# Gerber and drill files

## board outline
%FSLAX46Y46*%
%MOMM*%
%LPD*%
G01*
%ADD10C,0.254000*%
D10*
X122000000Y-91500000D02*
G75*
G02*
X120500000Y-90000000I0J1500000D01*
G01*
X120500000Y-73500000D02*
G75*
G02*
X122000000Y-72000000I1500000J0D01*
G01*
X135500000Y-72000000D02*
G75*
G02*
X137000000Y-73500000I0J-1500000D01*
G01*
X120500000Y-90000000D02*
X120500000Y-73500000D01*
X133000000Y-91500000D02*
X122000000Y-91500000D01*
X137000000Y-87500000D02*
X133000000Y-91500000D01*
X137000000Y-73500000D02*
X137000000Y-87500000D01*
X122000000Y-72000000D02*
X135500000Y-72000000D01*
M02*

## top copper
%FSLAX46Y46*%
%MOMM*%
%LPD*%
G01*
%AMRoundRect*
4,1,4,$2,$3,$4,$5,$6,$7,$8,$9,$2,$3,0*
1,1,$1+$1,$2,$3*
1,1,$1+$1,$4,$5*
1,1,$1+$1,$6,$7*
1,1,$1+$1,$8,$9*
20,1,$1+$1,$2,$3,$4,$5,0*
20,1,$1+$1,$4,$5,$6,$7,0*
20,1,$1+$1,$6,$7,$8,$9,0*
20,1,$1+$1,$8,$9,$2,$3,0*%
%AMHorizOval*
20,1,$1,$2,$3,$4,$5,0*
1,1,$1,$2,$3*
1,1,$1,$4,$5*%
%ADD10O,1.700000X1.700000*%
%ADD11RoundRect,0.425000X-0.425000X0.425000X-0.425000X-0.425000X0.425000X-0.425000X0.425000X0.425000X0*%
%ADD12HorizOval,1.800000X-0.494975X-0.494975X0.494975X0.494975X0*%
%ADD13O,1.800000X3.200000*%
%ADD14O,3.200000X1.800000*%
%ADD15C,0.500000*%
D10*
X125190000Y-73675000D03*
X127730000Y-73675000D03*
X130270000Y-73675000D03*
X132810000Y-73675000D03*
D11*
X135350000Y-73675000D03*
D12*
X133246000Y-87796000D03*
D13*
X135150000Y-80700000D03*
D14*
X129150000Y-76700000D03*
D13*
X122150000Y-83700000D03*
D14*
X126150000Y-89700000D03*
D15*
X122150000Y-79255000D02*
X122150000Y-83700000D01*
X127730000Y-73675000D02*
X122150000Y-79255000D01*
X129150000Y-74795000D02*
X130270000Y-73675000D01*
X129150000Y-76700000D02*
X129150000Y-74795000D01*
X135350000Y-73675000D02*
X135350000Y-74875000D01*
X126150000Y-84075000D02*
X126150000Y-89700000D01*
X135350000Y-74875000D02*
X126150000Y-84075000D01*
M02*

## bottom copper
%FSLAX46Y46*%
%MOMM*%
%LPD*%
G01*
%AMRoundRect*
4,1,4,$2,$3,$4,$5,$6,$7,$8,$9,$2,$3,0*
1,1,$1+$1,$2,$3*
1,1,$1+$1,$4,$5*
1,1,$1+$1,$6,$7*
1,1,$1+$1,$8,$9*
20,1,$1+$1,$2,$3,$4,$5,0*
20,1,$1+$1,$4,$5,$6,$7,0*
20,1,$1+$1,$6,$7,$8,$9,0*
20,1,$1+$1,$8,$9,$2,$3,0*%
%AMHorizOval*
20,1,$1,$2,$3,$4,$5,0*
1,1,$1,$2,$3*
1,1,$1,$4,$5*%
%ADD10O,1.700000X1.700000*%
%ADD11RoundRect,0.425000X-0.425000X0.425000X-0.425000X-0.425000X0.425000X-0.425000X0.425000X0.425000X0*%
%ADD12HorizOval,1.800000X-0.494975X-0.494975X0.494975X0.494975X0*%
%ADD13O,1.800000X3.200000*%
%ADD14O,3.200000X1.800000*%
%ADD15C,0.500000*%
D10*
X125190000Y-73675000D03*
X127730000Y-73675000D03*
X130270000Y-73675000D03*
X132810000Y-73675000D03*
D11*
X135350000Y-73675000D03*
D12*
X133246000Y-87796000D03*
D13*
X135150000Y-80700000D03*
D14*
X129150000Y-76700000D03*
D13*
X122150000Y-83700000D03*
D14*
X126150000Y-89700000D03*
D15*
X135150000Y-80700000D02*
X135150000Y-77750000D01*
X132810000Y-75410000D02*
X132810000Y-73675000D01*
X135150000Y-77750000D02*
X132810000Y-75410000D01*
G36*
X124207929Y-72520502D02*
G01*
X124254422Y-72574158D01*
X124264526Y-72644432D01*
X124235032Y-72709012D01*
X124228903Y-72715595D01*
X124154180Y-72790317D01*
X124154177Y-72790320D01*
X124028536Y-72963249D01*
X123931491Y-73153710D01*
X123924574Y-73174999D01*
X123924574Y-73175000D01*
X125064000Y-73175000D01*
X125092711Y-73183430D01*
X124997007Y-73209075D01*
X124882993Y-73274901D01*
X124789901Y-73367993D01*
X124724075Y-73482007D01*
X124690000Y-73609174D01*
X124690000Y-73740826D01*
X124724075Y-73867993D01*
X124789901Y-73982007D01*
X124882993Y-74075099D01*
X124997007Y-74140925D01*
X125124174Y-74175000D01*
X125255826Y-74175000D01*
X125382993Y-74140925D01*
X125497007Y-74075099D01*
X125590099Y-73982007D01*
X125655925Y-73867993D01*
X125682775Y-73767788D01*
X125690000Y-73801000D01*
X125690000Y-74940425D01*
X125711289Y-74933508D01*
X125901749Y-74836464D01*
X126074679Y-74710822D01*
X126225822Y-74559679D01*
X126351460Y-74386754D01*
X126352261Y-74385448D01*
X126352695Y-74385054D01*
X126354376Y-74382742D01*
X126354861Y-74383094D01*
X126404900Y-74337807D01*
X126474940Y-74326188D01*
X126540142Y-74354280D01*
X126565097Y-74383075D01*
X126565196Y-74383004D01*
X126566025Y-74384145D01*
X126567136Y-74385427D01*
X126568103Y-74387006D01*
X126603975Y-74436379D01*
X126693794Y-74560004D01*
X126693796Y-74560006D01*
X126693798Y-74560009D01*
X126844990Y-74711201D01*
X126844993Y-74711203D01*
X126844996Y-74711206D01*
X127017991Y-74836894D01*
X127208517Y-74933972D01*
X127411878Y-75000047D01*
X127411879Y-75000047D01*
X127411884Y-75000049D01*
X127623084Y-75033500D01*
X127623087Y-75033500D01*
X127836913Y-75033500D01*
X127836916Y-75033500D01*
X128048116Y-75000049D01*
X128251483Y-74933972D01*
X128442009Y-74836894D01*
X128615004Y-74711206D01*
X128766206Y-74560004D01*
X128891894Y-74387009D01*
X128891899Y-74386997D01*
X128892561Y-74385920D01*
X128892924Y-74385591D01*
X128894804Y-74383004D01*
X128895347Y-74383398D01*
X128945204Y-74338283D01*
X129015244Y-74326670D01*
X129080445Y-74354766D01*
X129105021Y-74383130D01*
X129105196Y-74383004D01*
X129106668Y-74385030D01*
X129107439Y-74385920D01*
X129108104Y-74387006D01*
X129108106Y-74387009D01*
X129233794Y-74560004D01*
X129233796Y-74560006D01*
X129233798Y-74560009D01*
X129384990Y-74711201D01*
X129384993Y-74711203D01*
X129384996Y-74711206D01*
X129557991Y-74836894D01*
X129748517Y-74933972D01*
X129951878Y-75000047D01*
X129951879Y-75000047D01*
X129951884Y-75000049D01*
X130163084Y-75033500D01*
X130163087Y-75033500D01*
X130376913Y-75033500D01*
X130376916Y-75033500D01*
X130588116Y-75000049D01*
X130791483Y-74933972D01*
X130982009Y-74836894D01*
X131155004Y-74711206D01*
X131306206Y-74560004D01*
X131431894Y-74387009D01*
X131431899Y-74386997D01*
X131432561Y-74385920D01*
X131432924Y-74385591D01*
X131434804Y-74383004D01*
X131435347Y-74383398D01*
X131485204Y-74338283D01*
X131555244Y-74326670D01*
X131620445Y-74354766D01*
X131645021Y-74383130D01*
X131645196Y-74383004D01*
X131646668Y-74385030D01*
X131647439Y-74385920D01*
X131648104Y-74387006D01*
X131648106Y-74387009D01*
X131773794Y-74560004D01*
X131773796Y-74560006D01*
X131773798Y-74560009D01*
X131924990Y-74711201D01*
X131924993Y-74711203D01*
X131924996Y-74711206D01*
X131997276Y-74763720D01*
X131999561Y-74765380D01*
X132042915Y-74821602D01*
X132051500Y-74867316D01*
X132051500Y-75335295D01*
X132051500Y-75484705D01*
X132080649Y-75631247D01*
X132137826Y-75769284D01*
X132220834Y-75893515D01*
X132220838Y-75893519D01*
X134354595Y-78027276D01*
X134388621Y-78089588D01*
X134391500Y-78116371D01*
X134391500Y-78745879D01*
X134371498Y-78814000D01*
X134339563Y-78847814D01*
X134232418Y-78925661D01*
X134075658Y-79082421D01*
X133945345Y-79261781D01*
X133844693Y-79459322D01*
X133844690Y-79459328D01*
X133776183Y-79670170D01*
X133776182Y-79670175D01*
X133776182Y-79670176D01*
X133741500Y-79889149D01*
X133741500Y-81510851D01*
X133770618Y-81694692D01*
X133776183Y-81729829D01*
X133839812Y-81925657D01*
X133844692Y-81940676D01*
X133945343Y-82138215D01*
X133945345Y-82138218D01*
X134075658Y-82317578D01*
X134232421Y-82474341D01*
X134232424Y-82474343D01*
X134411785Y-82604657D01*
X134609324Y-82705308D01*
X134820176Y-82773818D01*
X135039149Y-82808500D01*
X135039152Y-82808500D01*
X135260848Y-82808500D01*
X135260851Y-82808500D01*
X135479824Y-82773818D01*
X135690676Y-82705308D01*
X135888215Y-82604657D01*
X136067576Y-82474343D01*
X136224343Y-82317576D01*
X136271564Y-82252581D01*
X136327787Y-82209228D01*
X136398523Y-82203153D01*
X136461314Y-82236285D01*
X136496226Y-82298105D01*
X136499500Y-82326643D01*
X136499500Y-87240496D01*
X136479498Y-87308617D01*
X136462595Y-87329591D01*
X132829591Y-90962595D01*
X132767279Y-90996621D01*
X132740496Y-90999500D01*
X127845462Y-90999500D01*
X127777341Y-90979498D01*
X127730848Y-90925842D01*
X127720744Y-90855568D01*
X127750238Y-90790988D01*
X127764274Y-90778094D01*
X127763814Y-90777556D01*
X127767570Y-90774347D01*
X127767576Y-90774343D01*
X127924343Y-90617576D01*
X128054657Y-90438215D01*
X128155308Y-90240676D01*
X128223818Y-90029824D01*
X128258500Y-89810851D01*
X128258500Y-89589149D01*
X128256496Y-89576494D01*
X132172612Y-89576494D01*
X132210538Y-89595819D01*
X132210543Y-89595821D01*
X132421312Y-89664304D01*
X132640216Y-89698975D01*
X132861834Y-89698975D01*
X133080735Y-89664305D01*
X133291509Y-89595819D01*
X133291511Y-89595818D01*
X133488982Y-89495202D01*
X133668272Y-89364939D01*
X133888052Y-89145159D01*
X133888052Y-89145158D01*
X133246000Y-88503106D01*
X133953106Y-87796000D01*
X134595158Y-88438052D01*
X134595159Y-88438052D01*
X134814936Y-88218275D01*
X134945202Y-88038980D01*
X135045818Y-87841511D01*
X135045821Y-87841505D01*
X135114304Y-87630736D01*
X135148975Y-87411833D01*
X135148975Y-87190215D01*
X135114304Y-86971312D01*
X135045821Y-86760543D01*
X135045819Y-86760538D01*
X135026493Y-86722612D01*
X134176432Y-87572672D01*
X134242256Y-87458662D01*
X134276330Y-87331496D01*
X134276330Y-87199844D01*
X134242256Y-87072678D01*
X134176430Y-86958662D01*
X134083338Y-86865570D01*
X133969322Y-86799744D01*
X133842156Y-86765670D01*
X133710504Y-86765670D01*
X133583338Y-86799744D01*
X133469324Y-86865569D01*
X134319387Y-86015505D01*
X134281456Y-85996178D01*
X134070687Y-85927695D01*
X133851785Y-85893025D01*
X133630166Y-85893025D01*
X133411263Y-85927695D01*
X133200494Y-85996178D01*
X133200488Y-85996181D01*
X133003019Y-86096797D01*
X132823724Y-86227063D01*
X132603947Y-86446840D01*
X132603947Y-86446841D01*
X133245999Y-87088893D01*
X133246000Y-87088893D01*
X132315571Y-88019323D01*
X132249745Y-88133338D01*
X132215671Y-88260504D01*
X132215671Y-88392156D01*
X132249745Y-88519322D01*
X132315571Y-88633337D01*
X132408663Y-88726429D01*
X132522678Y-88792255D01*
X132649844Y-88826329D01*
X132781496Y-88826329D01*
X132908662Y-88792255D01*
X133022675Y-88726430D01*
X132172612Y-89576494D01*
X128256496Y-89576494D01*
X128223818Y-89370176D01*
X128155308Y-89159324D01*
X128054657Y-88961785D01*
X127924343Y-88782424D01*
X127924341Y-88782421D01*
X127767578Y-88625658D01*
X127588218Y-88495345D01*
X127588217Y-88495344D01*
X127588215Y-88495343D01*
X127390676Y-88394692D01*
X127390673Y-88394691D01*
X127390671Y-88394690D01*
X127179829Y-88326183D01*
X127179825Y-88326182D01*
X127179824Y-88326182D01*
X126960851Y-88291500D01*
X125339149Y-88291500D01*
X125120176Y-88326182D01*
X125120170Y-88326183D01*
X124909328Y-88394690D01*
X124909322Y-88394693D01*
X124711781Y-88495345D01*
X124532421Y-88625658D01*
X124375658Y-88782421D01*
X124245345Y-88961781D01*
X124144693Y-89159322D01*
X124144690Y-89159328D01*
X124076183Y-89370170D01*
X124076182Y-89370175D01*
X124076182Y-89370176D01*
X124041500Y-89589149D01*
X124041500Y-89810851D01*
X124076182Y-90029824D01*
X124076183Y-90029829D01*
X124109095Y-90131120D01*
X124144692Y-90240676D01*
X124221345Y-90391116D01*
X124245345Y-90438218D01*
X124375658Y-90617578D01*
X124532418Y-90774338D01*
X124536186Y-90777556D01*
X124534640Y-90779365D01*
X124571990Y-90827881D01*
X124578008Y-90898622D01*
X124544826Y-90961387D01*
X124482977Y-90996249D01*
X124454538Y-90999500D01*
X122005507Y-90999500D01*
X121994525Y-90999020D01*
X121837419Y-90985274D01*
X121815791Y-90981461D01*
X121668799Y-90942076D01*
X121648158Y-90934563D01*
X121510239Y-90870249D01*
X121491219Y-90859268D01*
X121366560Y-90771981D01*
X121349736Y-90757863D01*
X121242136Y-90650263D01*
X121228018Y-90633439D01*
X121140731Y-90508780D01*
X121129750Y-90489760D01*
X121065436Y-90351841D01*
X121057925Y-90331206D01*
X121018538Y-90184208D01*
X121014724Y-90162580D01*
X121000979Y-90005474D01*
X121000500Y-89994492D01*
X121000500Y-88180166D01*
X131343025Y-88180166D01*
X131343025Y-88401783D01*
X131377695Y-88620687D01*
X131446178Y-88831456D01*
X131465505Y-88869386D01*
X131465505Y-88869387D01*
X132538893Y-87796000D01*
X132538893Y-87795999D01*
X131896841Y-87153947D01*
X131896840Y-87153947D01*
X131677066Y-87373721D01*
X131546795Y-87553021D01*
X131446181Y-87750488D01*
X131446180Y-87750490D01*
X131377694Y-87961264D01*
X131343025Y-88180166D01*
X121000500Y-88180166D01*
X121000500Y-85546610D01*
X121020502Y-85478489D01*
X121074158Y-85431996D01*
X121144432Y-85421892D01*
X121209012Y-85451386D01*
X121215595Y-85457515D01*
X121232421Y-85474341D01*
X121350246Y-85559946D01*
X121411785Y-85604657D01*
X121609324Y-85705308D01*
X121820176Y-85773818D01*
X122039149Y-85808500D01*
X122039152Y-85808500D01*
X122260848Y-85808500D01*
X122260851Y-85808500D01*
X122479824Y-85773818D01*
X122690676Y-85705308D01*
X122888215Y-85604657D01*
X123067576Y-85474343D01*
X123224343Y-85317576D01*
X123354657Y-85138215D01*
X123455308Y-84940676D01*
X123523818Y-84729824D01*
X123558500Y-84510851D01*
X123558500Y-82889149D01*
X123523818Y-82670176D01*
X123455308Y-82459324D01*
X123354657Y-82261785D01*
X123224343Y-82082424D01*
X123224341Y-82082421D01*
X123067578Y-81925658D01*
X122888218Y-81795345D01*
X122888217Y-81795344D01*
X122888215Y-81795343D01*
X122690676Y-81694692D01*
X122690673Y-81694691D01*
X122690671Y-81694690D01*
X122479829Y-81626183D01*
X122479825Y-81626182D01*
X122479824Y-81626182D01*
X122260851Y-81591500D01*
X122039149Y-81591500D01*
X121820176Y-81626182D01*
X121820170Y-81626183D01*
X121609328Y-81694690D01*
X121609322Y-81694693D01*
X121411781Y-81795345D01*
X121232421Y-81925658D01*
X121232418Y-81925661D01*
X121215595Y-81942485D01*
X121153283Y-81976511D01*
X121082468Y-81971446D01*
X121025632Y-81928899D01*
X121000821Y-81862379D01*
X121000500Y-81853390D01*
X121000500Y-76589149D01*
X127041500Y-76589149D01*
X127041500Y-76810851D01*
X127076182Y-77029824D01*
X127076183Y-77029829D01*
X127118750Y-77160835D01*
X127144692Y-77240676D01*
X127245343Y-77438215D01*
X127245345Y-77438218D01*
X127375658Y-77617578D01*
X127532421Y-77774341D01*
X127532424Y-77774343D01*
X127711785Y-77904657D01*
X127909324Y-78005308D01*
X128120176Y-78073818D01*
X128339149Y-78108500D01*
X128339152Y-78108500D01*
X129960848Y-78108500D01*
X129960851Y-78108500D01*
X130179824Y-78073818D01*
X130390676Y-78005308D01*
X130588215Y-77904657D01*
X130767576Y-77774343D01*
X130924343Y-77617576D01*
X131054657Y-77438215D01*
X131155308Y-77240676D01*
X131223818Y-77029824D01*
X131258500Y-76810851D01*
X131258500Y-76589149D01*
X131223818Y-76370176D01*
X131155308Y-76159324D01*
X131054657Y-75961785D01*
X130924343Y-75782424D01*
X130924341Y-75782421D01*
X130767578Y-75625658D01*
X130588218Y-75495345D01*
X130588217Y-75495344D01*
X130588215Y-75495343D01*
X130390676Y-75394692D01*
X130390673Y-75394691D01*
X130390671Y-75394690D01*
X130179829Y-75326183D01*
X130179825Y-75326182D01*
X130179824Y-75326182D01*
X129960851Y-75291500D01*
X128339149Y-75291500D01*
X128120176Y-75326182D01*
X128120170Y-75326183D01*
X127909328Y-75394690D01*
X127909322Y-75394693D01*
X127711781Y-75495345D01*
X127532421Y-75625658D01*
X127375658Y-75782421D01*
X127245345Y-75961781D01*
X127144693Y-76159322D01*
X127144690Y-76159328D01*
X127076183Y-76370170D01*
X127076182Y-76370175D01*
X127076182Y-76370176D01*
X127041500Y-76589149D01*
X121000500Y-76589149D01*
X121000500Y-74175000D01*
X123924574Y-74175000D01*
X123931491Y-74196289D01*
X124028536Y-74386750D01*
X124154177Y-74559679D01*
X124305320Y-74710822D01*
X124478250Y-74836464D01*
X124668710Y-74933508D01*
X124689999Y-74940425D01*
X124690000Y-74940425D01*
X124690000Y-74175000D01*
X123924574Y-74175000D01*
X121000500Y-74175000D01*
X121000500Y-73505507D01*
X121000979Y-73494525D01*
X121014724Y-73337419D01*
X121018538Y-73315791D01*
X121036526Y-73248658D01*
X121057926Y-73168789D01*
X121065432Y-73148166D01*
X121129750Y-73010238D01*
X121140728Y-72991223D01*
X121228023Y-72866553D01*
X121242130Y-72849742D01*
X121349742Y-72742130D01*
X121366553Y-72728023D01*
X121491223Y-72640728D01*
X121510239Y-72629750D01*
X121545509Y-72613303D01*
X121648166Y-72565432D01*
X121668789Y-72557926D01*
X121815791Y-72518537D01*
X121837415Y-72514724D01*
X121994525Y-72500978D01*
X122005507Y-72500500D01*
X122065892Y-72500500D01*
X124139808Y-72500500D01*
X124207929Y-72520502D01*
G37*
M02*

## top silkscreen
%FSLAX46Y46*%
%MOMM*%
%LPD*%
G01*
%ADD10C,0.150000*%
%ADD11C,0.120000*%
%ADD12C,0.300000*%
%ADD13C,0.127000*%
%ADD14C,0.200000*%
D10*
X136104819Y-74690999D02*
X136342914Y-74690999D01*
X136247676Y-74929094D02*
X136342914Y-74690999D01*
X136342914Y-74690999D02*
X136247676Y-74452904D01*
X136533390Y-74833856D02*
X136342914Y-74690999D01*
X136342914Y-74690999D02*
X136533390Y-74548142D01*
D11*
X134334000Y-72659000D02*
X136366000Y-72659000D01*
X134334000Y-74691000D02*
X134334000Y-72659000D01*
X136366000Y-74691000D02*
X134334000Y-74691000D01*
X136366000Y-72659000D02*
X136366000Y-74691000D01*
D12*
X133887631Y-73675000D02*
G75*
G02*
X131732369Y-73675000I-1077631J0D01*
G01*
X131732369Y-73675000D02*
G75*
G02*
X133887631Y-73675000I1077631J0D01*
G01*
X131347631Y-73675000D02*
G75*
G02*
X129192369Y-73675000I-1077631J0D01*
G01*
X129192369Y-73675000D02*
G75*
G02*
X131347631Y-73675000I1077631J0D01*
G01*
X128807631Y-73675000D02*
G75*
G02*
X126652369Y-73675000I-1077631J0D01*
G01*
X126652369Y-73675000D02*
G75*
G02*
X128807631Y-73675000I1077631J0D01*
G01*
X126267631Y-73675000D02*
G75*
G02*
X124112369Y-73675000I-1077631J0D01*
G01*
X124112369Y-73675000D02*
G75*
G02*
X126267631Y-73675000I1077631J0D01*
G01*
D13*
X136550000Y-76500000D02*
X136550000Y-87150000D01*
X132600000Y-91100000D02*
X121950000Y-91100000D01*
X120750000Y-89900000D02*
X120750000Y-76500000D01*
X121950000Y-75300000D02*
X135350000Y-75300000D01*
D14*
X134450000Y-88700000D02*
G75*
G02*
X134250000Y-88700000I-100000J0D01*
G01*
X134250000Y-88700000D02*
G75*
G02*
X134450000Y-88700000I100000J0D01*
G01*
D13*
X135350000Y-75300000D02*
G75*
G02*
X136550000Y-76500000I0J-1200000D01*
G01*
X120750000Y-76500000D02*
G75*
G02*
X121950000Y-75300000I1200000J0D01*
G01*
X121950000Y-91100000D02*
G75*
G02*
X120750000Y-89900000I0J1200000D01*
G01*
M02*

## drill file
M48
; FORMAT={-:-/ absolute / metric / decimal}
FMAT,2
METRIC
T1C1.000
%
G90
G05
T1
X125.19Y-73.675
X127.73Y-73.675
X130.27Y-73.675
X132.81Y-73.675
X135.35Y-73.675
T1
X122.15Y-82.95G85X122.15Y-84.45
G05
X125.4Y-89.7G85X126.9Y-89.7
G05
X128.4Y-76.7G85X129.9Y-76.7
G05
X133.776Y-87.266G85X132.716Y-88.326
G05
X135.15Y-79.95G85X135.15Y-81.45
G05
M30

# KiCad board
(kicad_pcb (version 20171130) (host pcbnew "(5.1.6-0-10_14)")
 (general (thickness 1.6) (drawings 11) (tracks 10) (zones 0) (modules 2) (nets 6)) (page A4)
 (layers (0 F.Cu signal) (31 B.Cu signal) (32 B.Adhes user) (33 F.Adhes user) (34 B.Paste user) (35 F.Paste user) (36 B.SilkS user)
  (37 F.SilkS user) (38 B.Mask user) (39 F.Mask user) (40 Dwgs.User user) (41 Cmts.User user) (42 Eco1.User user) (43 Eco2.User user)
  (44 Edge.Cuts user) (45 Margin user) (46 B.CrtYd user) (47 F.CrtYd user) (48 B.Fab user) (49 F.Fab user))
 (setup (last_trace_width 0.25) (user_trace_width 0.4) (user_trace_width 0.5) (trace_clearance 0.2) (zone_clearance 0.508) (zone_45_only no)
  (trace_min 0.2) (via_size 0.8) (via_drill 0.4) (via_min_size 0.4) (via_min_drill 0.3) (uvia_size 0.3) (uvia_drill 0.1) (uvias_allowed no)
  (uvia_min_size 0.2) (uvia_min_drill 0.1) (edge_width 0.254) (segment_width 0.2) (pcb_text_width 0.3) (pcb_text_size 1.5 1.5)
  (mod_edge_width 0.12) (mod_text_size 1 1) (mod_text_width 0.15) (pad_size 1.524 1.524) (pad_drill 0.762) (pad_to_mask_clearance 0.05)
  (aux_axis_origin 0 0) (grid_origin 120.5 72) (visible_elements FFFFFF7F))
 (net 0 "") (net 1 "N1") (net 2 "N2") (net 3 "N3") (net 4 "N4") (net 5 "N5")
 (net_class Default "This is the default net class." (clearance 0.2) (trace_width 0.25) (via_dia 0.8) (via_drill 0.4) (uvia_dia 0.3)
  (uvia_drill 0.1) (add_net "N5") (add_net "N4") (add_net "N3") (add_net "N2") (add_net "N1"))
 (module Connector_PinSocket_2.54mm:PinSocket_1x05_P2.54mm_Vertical (layer F.Cu) (at 135.35 73.675 270)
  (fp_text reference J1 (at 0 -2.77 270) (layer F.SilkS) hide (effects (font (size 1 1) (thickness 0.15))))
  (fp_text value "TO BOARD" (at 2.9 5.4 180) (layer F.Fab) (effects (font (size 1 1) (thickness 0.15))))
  (fp_line (start -1.016 1.016) (end -1.016 -1.016) (layer F.SilkS) (width 0.12))
  (fp_line (start 1.016 1.016) (end -1.016 1.016) (layer F.SilkS) (width 0.12))
  (fp_line (start 1.016 -1.016) (end 1.016 1.016) (layer F.SilkS) (width 0.12))
  (fp_line (start -1.016 -1.016) (end 1.016 -1.016) (layer F.SilkS) (width 0.12))
  (fp_circle (center 0 2.54) (end 1.077631 2.54) (layer F.SilkS) (width 0.3))
  (fp_circle (center 0 5.08) (end 1.077631 5.08) (layer F.SilkS) (width 0.3))
  (fp_circle (center 0 7.62) (end 1.077631 7.62) (layer F.SilkS) (width 0.3))
  (fp_circle (center 0 10.16) (end 1.077631 10.16) (layer F.SilkS) (width 0.3))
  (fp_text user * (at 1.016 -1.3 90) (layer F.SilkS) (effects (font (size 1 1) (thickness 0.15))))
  (pad 5 thru_hole oval (at 0 10.16 270) (size 1.7 1.7) (drill 1) (layers *.Cu *.Mask) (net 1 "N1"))
  (pad 4 thru_hole oval (at 0 7.62 270) (size 1.7 1.7) (drill 1) (layers *.Cu *.Mask) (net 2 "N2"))
  (pad 3 thru_hole oval (at 0 5.08 270) (size 1.7 1.7) (drill 1) (layers *.Cu *.Mask) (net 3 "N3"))
  (pad 2 thru_hole oval (at 0 2.54 270) (size 1.7 1.7) (drill 1) (layers *.Cu *.Mask) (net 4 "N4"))
  (pad 1 thru_hole roundrect (at 0 0 270) (size 1.7 1.7) (drill 1) (layers *.Cu *.Mask) (roundrect_rratio 0.25) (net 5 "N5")))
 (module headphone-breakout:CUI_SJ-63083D (layer F.Cu) (at 128.65 83.2)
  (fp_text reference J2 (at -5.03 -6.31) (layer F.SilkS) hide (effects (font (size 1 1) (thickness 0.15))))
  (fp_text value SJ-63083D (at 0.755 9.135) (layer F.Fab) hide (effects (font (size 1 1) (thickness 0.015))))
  (fp_line (start 7.9 -6.7) (end 7.9 3.95) (layer F.SilkS) (width 0.127))
  (fp_line (start 3.95 7.9) (end -6.7 7.9) (layer F.SilkS) (width 0.127))
  (fp_line (start -7.9 6.7) (end -7.9 -6.7) (layer F.SilkS) (width 0.127))
  (fp_line (start -6.7 -7.9) (end 6.7 -7.9) (layer F.SilkS) (width 0.127))
  (fp_circle (center 5.7 5.5) (end 5.8 5.5) (layer F.SilkS) (width 0.2))
  (fp_arc (start 6.7 -6.7) (end 7.9 -6.7) (angle -90) (layer F.SilkS) (width 0.127))
  (fp_arc (start -6.7 -6.7) (end -6.7 -7.9) (angle -90) (layer F.SilkS) (width 0.127))
  (fp_arc (start -6.7 6.7) (end -7.9 6.7) (angle -90) (layer F.SilkS) (width 0.127))
  (pad S thru_hole oval (at 4.596 4.596 315) (size 1.8 3.2) (drill oval 1 2.5) (layers *.Cu *.Mask) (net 1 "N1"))
  (pad TN thru_hole oval (at 6.5 -2.5) (size 1.8 3.2) (drill oval 1 2.5) (layers *.Cu *.Mask) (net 4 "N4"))
  (pad T thru_hole oval (at 0.5 -6.5) (size 3.2 1.8) (drill oval 2.5 1) (layers *.Cu *.Mask) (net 3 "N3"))
  (pad R thru_hole oval (at -6.5 0.5) (size 1.8 3.2) (drill oval 1 2.5) (layers *.Cu *.Mask) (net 2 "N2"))
  (pad RN thru_hole oval (at -2.5 6.5) (size 3.2 1.8) (drill oval 2.5 1) (layers *.Cu *.Mask) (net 5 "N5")))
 (gr_arc (start 122 90) (end 120.5 90) (angle -90) (layer Edge.Cuts) (width 0.254))
 (gr_arc (start 122 73.5) (end 122 72) (angle -90) (layer Edge.Cuts) (width 0.254))
 (gr_arc (start 135.5 73.5) (end 137 73.5) (angle -90) (layer Edge.Cuts) (width 0.254))
 (gr_line (start 120.5 90) (end 120.5 73.5) (layer Edge.Cuts) (width 0.254))
 (gr_line (start 133 91.5) (end 122 91.5) (layer Edge.Cuts) (width 0.254))
 (gr_line (start 137 87.5) (end 133 91.5) (layer Edge.Cuts) (width 0.254))
 (gr_line (start 137 73.5) (end 137 87.5) (layer Edge.Cuts) (width 0.254))
 (gr_line (start 122 72) (end 135.5 72) (layer Edge.Cuts) (width 0.254))
 (segment (start 122.15 79.255) (end 122.15 83.7) (width 0.5) (layer F.Cu) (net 2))
 (segment (start 127.73 73.675) (end 122.15 79.255) (width 0.5) (layer F.Cu) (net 2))
 (segment (start 129.15 74.795) (end 130.27 73.675) (width 0.5) (layer F.Cu) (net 3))
 (segment (start 129.15 76.7) (end 129.15 74.795) (width 0.5) (layer F.Cu) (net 3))
 (segment (start 135.15 80.7) (end 135.15 77.75) (width 0.5) (layer B.Cu) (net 4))
 (segment (start 132.81 75.41) (end 132.81 73.675) (width 0.5) (layer B.Cu) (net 4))
 (segment (start 135.15 77.75) (end 132.81 75.41) (width 0.5) (layer B.Cu) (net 4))
 (segment (start 135.35 73.675) (end 135.35 74.875) (width 0.5) (layer F.Cu) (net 5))
 (segment (start 126.15 84.075) (end 126.15 89.7) (width 0.5) (layer F.Cu) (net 5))
 (segment (start 135.35 74.875) (end 126.15 84.075) (width 0.5) (layer F.Cu) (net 5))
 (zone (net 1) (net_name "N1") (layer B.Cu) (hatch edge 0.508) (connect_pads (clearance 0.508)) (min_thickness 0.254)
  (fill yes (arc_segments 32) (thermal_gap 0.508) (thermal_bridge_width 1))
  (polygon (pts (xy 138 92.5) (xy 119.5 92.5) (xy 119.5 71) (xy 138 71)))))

